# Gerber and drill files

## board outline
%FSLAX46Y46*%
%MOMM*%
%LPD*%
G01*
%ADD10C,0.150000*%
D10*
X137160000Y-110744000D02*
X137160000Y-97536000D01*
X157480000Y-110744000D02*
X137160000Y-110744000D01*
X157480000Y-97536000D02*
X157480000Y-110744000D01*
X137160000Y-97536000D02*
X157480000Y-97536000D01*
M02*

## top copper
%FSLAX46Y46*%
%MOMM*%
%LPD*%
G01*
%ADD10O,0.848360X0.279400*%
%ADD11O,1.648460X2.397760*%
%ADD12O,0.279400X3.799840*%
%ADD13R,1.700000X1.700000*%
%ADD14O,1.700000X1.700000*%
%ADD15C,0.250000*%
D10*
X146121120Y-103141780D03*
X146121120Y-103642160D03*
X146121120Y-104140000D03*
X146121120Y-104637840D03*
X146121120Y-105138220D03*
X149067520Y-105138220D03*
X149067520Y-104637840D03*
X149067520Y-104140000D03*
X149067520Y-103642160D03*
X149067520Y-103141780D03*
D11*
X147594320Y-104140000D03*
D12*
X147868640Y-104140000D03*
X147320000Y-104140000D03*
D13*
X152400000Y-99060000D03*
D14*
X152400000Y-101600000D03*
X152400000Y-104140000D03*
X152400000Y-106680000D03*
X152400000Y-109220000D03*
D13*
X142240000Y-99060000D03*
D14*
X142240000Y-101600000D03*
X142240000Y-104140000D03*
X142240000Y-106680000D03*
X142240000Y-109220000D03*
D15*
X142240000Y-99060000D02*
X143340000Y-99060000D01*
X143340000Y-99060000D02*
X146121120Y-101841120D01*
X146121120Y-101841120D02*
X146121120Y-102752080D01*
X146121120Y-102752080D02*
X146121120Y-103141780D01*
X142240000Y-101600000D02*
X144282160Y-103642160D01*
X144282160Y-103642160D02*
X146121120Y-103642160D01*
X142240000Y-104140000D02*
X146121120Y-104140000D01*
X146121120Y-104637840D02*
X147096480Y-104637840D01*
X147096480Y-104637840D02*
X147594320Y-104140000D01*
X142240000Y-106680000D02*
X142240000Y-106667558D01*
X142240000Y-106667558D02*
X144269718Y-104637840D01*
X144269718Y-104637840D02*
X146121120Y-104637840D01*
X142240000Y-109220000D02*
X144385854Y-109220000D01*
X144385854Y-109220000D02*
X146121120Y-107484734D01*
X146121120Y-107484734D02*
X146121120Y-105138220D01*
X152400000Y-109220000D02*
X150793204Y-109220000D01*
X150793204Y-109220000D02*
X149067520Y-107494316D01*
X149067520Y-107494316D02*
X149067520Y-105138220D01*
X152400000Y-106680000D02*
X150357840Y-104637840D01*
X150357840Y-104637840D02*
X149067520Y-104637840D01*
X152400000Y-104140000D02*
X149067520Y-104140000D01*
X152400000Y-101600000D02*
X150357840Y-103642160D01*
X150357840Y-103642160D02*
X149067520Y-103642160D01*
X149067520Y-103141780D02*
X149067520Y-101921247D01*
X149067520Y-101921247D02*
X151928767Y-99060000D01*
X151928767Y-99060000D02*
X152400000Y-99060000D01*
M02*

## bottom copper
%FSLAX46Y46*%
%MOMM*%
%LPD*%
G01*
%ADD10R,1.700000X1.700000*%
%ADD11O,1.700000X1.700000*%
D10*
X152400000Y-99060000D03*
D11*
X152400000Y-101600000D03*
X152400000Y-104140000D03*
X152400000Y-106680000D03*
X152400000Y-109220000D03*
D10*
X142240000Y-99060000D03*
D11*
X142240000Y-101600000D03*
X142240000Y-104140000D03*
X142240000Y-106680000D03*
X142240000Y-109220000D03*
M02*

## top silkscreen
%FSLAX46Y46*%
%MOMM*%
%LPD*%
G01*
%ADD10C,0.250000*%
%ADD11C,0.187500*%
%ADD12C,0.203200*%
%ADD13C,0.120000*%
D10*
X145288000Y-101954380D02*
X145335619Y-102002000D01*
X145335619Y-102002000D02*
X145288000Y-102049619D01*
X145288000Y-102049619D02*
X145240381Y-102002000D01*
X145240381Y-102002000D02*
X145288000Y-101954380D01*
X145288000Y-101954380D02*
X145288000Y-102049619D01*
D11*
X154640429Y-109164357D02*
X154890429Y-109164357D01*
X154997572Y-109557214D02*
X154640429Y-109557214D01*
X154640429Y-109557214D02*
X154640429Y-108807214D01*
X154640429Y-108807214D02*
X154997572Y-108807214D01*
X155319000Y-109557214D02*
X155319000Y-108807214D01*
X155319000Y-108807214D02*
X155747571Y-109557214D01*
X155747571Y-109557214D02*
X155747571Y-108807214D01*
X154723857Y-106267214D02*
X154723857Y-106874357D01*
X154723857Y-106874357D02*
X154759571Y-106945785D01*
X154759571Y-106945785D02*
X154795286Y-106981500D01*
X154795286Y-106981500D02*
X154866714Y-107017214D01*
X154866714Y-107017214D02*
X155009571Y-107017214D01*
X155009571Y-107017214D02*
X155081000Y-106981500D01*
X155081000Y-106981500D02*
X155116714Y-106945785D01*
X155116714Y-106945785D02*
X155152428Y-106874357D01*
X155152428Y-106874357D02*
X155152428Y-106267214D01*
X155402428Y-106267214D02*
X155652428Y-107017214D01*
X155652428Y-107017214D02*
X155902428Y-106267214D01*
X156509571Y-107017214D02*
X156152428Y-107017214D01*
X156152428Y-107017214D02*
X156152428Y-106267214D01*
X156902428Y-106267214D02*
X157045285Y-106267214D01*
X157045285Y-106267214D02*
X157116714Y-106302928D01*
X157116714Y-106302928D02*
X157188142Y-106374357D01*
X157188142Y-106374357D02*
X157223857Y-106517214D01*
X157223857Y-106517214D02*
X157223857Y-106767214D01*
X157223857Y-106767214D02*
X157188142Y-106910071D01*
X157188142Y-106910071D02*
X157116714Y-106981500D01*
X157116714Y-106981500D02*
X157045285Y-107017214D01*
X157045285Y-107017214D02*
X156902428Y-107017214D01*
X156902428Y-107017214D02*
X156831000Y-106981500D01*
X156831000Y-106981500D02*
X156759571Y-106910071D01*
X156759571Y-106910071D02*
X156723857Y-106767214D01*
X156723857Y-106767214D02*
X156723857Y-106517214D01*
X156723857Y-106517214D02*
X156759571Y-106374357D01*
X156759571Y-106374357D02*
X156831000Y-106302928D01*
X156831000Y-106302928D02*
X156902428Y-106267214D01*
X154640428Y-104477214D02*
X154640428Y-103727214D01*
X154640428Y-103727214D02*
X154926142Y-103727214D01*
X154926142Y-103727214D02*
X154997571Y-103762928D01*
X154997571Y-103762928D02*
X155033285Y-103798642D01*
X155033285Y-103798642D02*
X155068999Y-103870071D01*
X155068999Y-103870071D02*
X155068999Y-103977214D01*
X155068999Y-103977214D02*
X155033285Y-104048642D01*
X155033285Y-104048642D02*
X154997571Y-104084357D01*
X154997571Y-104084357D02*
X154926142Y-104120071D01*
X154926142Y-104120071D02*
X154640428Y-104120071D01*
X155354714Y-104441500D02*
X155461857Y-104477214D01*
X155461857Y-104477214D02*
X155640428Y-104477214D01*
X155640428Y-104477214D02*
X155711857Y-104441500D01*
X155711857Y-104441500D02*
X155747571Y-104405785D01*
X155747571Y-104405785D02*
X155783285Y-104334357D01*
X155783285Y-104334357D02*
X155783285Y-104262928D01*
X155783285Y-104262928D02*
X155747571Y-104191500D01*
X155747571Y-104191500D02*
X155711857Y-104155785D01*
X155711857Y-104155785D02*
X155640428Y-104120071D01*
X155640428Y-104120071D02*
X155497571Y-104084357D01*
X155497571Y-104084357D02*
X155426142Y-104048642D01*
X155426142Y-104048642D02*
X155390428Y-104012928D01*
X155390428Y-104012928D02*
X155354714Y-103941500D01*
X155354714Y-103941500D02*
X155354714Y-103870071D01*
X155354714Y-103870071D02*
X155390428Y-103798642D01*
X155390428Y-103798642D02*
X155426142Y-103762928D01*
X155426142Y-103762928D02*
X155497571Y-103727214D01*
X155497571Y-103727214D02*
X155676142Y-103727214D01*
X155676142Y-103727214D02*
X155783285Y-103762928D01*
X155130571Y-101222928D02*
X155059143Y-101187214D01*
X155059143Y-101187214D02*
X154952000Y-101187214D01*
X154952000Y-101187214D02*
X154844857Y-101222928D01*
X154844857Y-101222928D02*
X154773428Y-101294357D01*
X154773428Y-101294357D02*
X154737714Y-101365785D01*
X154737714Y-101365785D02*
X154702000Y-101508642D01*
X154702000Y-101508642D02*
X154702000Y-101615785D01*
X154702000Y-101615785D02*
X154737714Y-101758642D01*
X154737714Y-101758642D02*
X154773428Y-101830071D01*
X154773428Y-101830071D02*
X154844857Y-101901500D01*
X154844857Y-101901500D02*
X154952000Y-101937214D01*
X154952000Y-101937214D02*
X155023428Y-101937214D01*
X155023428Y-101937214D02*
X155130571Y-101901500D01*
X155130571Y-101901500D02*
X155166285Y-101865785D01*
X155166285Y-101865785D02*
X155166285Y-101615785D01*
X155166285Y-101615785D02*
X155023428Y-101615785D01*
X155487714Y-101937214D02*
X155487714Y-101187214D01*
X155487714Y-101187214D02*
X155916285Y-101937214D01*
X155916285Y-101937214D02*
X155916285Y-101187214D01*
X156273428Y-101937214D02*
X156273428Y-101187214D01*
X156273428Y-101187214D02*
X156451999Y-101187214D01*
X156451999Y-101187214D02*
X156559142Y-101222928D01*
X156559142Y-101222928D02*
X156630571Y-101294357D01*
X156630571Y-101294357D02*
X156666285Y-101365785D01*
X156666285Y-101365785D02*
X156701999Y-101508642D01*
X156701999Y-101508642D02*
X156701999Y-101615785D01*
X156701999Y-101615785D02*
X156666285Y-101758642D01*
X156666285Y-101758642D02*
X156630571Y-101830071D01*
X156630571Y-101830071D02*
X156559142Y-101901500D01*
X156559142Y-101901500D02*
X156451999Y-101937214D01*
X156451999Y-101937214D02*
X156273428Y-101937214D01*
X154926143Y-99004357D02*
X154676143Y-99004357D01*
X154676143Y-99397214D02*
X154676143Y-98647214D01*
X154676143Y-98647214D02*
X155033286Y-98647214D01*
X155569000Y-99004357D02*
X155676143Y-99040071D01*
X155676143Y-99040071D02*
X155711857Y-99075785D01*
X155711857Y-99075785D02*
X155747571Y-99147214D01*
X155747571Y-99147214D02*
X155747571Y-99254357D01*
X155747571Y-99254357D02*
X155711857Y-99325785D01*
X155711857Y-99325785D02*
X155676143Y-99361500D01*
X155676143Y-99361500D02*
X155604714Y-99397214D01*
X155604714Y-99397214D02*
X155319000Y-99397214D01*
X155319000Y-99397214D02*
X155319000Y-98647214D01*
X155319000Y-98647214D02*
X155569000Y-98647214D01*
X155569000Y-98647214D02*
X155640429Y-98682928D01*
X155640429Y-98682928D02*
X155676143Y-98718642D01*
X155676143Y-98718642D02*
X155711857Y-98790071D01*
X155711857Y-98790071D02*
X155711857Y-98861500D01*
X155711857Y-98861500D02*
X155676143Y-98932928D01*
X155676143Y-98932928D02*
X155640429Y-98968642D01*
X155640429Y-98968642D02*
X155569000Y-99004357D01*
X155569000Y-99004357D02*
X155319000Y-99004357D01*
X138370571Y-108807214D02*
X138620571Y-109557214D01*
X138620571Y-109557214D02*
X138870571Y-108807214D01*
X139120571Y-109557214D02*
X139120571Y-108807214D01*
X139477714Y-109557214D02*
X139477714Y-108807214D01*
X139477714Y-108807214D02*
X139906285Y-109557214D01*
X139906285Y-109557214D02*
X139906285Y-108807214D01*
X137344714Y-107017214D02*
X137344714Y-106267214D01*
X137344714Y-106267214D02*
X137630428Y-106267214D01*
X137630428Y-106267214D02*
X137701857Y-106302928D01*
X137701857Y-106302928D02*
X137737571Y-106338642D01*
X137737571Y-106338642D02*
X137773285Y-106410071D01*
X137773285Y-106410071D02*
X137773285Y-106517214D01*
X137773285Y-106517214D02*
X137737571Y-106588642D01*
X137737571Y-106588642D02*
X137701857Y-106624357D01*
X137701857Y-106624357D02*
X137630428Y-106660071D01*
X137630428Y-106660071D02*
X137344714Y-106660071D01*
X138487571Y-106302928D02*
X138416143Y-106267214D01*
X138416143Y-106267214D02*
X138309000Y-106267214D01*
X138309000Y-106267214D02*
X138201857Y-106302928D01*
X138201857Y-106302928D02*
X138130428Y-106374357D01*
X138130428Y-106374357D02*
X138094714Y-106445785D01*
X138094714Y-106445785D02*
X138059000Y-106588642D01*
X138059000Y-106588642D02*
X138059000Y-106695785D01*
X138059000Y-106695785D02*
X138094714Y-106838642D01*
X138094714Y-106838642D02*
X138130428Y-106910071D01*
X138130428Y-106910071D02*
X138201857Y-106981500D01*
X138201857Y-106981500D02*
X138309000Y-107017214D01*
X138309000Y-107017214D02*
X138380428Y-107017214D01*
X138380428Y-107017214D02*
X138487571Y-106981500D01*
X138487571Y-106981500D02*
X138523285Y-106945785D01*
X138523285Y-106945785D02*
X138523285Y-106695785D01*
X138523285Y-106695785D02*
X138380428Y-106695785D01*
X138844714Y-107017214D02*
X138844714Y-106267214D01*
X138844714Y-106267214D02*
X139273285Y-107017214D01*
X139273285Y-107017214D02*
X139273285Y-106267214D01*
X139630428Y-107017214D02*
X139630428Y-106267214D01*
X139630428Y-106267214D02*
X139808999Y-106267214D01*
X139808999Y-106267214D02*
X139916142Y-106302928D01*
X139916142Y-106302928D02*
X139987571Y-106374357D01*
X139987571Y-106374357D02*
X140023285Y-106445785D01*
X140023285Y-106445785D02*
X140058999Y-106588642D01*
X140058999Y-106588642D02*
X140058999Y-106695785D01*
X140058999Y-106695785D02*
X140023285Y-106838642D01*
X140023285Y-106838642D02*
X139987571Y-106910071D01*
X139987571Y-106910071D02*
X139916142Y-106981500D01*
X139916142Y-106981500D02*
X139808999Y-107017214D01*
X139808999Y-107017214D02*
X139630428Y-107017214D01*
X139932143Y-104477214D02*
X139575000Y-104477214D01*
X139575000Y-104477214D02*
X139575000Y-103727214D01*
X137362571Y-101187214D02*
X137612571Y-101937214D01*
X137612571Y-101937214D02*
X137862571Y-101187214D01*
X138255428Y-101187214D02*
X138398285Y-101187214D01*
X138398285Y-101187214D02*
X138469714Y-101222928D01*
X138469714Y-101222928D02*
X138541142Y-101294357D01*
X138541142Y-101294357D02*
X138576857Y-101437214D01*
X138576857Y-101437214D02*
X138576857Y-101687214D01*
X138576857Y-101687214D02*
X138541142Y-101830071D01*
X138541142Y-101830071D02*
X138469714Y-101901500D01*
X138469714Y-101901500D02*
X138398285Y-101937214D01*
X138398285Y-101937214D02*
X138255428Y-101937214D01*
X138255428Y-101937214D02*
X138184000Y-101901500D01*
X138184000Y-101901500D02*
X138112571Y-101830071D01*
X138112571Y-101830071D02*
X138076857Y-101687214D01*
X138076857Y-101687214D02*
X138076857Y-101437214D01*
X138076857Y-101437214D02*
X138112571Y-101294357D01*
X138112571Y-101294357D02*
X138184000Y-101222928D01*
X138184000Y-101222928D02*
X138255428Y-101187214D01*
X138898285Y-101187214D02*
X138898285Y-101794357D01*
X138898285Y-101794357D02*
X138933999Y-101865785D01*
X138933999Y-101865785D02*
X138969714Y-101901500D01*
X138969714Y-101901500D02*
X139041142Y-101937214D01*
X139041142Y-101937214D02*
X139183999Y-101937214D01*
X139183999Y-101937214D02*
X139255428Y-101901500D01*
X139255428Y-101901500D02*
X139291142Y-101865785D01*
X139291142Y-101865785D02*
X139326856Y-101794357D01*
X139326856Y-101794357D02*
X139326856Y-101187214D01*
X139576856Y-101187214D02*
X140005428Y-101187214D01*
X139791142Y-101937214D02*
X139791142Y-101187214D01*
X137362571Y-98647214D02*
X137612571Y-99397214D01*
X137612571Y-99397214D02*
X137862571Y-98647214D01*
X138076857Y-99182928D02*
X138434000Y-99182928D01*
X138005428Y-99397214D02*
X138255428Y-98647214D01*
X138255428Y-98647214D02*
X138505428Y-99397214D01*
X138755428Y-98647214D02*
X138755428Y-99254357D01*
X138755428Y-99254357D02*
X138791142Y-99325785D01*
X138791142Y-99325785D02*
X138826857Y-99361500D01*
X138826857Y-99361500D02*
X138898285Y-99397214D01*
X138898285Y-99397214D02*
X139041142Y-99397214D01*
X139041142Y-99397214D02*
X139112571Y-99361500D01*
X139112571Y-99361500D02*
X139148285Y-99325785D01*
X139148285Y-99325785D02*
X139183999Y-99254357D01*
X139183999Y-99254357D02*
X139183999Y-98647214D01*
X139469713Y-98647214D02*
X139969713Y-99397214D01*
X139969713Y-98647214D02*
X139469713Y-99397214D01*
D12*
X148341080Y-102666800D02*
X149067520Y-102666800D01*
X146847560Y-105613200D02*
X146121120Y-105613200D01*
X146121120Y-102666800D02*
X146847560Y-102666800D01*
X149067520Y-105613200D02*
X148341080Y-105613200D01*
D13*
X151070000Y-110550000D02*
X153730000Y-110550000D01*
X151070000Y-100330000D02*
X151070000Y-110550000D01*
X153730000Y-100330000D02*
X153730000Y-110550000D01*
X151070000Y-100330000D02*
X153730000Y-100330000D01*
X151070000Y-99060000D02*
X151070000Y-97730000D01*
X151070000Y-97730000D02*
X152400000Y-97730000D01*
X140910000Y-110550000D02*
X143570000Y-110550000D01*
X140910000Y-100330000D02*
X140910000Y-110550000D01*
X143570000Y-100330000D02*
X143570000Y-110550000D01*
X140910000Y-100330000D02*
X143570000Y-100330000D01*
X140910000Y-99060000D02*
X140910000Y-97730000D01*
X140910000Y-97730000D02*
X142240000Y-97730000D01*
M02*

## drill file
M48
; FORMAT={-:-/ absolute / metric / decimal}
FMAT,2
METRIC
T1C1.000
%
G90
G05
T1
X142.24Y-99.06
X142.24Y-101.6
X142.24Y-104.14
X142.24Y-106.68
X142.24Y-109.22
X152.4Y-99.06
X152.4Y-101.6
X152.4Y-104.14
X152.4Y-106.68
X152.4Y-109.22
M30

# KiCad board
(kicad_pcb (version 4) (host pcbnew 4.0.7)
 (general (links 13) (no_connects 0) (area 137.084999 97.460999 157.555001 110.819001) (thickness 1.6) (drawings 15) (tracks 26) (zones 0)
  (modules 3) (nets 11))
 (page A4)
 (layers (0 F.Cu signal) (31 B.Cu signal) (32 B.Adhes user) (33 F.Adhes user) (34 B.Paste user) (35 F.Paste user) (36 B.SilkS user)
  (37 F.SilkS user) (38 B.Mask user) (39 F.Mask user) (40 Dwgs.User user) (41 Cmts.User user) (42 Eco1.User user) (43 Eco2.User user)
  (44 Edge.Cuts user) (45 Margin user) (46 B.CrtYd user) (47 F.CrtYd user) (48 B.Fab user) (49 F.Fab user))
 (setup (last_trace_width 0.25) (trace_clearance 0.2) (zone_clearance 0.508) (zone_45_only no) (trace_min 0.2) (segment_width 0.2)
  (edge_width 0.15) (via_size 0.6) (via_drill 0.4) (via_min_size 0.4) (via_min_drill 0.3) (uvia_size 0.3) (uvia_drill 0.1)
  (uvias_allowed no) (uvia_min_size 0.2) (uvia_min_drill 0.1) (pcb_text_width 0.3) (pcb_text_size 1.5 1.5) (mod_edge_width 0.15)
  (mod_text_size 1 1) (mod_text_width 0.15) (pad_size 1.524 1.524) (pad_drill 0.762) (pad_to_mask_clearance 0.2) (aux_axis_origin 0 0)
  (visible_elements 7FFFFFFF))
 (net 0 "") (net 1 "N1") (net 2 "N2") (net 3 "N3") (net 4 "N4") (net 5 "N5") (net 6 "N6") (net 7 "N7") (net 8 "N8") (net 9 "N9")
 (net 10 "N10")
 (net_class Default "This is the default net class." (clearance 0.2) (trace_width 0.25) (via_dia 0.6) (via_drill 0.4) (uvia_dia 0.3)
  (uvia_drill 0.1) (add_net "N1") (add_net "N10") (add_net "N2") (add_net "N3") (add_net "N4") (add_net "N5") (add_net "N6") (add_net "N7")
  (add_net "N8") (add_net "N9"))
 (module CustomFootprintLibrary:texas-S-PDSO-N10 (layer F.Cu) (at 147.59432 104.14 270)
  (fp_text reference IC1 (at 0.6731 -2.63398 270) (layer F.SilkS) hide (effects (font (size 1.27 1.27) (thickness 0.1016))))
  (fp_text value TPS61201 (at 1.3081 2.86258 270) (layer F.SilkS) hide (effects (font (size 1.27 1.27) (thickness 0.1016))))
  (fp_line (start -1.4732 -0.74676) (end -1.4732 -1.4732) (layer F.SilkS) (width 0.2032))
  (fp_line (start 1.4732 0.74676) (end 1.4732 1.4732) (layer F.SilkS) (width 0.2032))
  (fp_line (start -1.4732 1.4732) (end -1.4732 0.74676) (layer F.SilkS) (width 0.2032))
  (fp_line (start 1.4732 -1.4732) (end 1.4732 -0.74676) (layer F.SilkS) (width 0.2032))
  (pad 1 smd oval (at -0.99822 1.4732) (size 0.84836 0.2794) (layers F.Cu F.Paste F.Mask) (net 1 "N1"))
  (pad 2 smd oval (at -0.49784 1.4732) (size 0.84836 0.2794) (layers F.Cu F.Paste F.Mask) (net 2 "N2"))
  (pad 3 smd oval (at 0 1.4732) (size 0.84836 0.2794) (layers F.Cu F.Paste F.Mask) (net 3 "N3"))
  (pad 4 smd oval (at 0.49784 1.4732) (size 0.84836 0.2794) (layers F.Cu F.Paste F.Mask) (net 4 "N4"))
  (pad 5 smd oval (at 0.99822 1.4732) (size 0.84836 0.2794) (layers F.Cu F.Paste F.Mask) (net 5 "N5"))
  (pad 6 smd oval (at 0.99822 -1.4732 180) (size 0.84836 0.2794) (layers F.Cu F.Paste F.Mask) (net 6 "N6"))
  (pad 7 smd oval (at 0.49784 -1.4732 180) (size 0.84836 0.2794) (layers F.Cu F.Paste F.Mask) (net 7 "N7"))
  (pad 8 smd oval (at 0 -1.4732 180) (size 0.84836 0.2794) (layers F.Cu F.Paste F.Mask) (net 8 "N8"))
  (pad 9 smd oval (at -0.49784 -1.4732 180) (size 0.84836 0.2794) (layers F.Cu F.Paste F.Mask) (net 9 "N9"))
  (pad 10 smd oval (at -0.99822 -1.4732 180) (size 0.84836 0.2794) (layers F.Cu F.Paste F.Mask) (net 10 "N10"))
  (pad PP smd oval (at 0 0 270) (size 2.39776 1.64846) (layers F.Cu F.Paste F.Mask) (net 4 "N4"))
  (pad PP@1 smd oval (at 0 -0.27432 270) (size 3.79984 0.2794) (layers F.Cu F.Paste F.Mask) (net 4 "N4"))
  (pad PP@2 smd oval (at 0 0.27432 270) (size 3.79984 0.2794) (layers F.Cu F.Paste F.Mask) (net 4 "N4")))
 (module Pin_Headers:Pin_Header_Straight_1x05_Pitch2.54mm (layer F.Cu) (at 152.4 99.06)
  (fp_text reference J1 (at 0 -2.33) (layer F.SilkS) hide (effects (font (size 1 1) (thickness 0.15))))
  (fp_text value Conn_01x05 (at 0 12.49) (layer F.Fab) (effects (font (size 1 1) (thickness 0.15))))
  (fp_line (start -1.33 11.49) (end 1.33 11.49) (layer F.SilkS) (width 0.12))
  (fp_line (start -1.33 1.27) (end -1.33 11.49) (layer F.SilkS) (width 0.12))
  (fp_line (start 1.33 1.27) (end 1.33 11.49) (layer F.SilkS) (width 0.12))
  (fp_line (start -1.33 1.27) (end 1.33 1.27) (layer F.SilkS) (width 0.12))
  (fp_line (start -1.33 0) (end -1.33 -1.33) (layer F.SilkS) (width 0.12))
  (fp_line (start -1.33 -1.33) (end 0 -1.33) (layer F.SilkS) (width 0.12))
  (pad 1 thru_hole rect (at 0 0) (size 1.7 1.7) (drill 1) (layers *.Cu *.Mask) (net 10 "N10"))
  (pad 2 thru_hole oval (at 0 2.54) (size 1.7 1.7) (drill 1) (layers *.Cu *.Mask) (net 9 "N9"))
  (pad 3 thru_hole oval (at 0 5.08) (size 1.7 1.7) (drill 1) (layers *.Cu *.Mask) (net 8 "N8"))
  (pad 4 thru_hole oval (at 0 7.62) (size 1.7 1.7) (drill 1) (layers *.Cu *.Mask) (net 7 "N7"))
  (pad 5 thru_hole oval (at 0 10.16) (size 1.7 1.7) (drill 1) (layers *.Cu *.Mask) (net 6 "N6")))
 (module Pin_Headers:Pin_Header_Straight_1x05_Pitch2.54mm (layer F.Cu) (at 142.24 99.06)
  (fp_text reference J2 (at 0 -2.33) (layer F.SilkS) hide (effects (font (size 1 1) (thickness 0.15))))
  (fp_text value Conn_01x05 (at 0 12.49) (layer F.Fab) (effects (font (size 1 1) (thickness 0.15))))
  (fp_line (start -1.33 11.49) (end 1.33 11.49) (layer F.SilkS) (width 0.12))
  (fp_line (start -1.33 1.27) (end -1.33 11.49) (layer F.SilkS) (width 0.12))
  (fp_line (start 1.33 1.27) (end 1.33 11.49) (layer F.SilkS) (width 0.12))
  (fp_line (start -1.33 1.27) (end 1.33 1.27) (layer F.SilkS) (width 0.12))
  (fp_line (start -1.33 0) (end -1.33 -1.33) (layer F.SilkS) (width 0.12))
  (fp_line (start -1.33 -1.33) (end 0 -1.33) (layer F.SilkS) (width 0.12))
  (pad 1 thru_hole rect (at 0 0) (size 1.7 1.7) (drill 1) (layers *.Cu *.Mask) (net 1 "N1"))
  (pad 2 thru_hole oval (at 0 2.54) (size 1.7 1.7) (drill 1) (layers *.Cu *.Mask) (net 2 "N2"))
  (pad 3 thru_hole oval (at 0 5.08) (size 1.7 1.7) (drill 1) (layers *.Cu *.Mask) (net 3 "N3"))
  (pad 4 thru_hole oval (at 0 7.62) (size 1.7 1.7) (drill 1) (layers *.Cu *.Mask) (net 4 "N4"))
  (pad 5 thru_hole oval (at 0 10.16) (size 1.7 1.7) (drill 1) (layers *.Cu *.Mask) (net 5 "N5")))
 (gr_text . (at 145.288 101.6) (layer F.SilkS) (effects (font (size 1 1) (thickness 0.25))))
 (gr_line (start 137.16 110.744) (end 137.16 97.536) (layer Edge.Cuts) (width 0.15))
 (gr_line (start 157.48 110.744) (end 137.16 110.744) (layer Edge.Cuts) (width 0.15))
 (gr_line (start 157.48 97.536) (end 157.48 110.744) (layer Edge.Cuts) (width 0.15))
 (gr_line (start 137.16 97.536) (end 157.48 97.536) (layer Edge.Cuts) (width 0.15))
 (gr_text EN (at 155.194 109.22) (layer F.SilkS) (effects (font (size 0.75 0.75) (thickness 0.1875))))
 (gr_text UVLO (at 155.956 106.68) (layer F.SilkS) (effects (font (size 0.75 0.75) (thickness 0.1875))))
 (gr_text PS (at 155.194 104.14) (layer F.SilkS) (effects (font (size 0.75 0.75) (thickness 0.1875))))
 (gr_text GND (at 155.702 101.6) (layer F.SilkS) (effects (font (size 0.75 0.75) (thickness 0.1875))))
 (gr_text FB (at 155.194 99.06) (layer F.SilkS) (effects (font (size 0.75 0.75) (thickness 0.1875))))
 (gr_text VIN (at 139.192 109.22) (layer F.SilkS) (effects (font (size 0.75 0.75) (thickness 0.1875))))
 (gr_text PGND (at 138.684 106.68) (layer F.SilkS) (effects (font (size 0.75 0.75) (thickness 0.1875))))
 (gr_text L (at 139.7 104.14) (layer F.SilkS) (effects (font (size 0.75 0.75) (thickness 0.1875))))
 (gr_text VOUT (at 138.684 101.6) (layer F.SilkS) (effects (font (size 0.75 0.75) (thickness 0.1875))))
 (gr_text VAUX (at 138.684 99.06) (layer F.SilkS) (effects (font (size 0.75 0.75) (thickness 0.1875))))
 (segment (start 142.24 99.06) (end 143.34 99.06) (width 0.25) (layer F.Cu) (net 1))
 (segment (start 143.34 99.06) (end 146.12112 101.84112) (width 0.25) (layer F.Cu) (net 1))
 (segment (start 146.12112 101.84112) (end 146.12112 102.75208) (width 0.25) (layer F.Cu) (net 1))
 (segment (start 146.12112 102.75208) (end 146.12112 103.14178) (width 0.25) (layer F.Cu) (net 1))
 (segment (start 142.24 101.6) (end 144.28216 103.64216) (width 0.25) (layer F.Cu) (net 2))
 (segment (start 144.28216 103.64216) (end 146.12112 103.64216) (width 0.25) (layer F.Cu) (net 2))
 (segment (start 142.24 104.14) (end 146.12112 104.14) (width 0.25) (layer F.Cu) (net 3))
 (segment (start 146.12112 104.63784) (end 147.09648 104.63784) (width 0.25) (layer F.Cu) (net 4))
 (segment (start 147.09648 104.63784) (end 147.59432 104.14) (width 0.25) (layer F.Cu) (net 4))
 (segment (start 142.24 106.68) (end 142.24 106.667558) (width 0.25) (layer F.Cu) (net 4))
 (segment (start 142.24 106.667558) (end 144.269718 104.63784) (width 0.25) (layer F.Cu) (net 4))
 (segment (start 144.269718 104.63784) (end 146.12112 104.63784) (width 0.25) (layer F.Cu) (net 4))
 (segment (start 142.24 109.22) (end 144.385854 109.22) (width 0.25) (layer F.Cu) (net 5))
 (segment (start 144.385854 109.22) (end 146.12112 107.484734) (width 0.25) (layer F.Cu) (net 5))
 (segment (start 146.12112 107.484734) (end 146.12112 105.13822) (width 0.25) (layer F.Cu) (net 5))
 (segment (start 152.4 109.22) (end 150.793204 109.22) (width 0.25) (layer F.Cu) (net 6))
 (segment (start 150.793204 109.22) (end 149.06752 107.494316) (width 0.25) (layer F.Cu) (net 6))
 (segment (start 149.06752 107.494316) (end 149.06752 105.13822) (width 0.25) (layer F.Cu) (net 6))
 (segment (start 152.4 106.68) (end 150.35784 104.63784) (width 0.25) (layer F.Cu) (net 7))
 (segment (start 150.35784 104.63784) (end 149.06752 104.63784) (width 0.25) (layer F.Cu) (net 7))
 (segment (start 152.4 104.14) (end 149.06752 104.14) (width 0.25) (layer F.Cu) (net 8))
 (segment (start 152.4 101.6) (end 150.35784 103.64216) (width 0.25) (layer F.Cu) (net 9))
 (segment (start 150.35784 103.64216) (end 149.06752 103.64216) (width 0.25) (layer F.Cu) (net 9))
 (segment (start 149.06752 103.14178) (end 149.06752 101.921247) (width 0.25) (layer F.Cu) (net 10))
 (segment (start 149.06752 101.921247) (end 151.928767 99.06) (width 0.25) (layer F.Cu) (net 10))
 (segment (start 151.928767 99.06) (end 152.4 99.06) (width 0.25) (layer F.Cu) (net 10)))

